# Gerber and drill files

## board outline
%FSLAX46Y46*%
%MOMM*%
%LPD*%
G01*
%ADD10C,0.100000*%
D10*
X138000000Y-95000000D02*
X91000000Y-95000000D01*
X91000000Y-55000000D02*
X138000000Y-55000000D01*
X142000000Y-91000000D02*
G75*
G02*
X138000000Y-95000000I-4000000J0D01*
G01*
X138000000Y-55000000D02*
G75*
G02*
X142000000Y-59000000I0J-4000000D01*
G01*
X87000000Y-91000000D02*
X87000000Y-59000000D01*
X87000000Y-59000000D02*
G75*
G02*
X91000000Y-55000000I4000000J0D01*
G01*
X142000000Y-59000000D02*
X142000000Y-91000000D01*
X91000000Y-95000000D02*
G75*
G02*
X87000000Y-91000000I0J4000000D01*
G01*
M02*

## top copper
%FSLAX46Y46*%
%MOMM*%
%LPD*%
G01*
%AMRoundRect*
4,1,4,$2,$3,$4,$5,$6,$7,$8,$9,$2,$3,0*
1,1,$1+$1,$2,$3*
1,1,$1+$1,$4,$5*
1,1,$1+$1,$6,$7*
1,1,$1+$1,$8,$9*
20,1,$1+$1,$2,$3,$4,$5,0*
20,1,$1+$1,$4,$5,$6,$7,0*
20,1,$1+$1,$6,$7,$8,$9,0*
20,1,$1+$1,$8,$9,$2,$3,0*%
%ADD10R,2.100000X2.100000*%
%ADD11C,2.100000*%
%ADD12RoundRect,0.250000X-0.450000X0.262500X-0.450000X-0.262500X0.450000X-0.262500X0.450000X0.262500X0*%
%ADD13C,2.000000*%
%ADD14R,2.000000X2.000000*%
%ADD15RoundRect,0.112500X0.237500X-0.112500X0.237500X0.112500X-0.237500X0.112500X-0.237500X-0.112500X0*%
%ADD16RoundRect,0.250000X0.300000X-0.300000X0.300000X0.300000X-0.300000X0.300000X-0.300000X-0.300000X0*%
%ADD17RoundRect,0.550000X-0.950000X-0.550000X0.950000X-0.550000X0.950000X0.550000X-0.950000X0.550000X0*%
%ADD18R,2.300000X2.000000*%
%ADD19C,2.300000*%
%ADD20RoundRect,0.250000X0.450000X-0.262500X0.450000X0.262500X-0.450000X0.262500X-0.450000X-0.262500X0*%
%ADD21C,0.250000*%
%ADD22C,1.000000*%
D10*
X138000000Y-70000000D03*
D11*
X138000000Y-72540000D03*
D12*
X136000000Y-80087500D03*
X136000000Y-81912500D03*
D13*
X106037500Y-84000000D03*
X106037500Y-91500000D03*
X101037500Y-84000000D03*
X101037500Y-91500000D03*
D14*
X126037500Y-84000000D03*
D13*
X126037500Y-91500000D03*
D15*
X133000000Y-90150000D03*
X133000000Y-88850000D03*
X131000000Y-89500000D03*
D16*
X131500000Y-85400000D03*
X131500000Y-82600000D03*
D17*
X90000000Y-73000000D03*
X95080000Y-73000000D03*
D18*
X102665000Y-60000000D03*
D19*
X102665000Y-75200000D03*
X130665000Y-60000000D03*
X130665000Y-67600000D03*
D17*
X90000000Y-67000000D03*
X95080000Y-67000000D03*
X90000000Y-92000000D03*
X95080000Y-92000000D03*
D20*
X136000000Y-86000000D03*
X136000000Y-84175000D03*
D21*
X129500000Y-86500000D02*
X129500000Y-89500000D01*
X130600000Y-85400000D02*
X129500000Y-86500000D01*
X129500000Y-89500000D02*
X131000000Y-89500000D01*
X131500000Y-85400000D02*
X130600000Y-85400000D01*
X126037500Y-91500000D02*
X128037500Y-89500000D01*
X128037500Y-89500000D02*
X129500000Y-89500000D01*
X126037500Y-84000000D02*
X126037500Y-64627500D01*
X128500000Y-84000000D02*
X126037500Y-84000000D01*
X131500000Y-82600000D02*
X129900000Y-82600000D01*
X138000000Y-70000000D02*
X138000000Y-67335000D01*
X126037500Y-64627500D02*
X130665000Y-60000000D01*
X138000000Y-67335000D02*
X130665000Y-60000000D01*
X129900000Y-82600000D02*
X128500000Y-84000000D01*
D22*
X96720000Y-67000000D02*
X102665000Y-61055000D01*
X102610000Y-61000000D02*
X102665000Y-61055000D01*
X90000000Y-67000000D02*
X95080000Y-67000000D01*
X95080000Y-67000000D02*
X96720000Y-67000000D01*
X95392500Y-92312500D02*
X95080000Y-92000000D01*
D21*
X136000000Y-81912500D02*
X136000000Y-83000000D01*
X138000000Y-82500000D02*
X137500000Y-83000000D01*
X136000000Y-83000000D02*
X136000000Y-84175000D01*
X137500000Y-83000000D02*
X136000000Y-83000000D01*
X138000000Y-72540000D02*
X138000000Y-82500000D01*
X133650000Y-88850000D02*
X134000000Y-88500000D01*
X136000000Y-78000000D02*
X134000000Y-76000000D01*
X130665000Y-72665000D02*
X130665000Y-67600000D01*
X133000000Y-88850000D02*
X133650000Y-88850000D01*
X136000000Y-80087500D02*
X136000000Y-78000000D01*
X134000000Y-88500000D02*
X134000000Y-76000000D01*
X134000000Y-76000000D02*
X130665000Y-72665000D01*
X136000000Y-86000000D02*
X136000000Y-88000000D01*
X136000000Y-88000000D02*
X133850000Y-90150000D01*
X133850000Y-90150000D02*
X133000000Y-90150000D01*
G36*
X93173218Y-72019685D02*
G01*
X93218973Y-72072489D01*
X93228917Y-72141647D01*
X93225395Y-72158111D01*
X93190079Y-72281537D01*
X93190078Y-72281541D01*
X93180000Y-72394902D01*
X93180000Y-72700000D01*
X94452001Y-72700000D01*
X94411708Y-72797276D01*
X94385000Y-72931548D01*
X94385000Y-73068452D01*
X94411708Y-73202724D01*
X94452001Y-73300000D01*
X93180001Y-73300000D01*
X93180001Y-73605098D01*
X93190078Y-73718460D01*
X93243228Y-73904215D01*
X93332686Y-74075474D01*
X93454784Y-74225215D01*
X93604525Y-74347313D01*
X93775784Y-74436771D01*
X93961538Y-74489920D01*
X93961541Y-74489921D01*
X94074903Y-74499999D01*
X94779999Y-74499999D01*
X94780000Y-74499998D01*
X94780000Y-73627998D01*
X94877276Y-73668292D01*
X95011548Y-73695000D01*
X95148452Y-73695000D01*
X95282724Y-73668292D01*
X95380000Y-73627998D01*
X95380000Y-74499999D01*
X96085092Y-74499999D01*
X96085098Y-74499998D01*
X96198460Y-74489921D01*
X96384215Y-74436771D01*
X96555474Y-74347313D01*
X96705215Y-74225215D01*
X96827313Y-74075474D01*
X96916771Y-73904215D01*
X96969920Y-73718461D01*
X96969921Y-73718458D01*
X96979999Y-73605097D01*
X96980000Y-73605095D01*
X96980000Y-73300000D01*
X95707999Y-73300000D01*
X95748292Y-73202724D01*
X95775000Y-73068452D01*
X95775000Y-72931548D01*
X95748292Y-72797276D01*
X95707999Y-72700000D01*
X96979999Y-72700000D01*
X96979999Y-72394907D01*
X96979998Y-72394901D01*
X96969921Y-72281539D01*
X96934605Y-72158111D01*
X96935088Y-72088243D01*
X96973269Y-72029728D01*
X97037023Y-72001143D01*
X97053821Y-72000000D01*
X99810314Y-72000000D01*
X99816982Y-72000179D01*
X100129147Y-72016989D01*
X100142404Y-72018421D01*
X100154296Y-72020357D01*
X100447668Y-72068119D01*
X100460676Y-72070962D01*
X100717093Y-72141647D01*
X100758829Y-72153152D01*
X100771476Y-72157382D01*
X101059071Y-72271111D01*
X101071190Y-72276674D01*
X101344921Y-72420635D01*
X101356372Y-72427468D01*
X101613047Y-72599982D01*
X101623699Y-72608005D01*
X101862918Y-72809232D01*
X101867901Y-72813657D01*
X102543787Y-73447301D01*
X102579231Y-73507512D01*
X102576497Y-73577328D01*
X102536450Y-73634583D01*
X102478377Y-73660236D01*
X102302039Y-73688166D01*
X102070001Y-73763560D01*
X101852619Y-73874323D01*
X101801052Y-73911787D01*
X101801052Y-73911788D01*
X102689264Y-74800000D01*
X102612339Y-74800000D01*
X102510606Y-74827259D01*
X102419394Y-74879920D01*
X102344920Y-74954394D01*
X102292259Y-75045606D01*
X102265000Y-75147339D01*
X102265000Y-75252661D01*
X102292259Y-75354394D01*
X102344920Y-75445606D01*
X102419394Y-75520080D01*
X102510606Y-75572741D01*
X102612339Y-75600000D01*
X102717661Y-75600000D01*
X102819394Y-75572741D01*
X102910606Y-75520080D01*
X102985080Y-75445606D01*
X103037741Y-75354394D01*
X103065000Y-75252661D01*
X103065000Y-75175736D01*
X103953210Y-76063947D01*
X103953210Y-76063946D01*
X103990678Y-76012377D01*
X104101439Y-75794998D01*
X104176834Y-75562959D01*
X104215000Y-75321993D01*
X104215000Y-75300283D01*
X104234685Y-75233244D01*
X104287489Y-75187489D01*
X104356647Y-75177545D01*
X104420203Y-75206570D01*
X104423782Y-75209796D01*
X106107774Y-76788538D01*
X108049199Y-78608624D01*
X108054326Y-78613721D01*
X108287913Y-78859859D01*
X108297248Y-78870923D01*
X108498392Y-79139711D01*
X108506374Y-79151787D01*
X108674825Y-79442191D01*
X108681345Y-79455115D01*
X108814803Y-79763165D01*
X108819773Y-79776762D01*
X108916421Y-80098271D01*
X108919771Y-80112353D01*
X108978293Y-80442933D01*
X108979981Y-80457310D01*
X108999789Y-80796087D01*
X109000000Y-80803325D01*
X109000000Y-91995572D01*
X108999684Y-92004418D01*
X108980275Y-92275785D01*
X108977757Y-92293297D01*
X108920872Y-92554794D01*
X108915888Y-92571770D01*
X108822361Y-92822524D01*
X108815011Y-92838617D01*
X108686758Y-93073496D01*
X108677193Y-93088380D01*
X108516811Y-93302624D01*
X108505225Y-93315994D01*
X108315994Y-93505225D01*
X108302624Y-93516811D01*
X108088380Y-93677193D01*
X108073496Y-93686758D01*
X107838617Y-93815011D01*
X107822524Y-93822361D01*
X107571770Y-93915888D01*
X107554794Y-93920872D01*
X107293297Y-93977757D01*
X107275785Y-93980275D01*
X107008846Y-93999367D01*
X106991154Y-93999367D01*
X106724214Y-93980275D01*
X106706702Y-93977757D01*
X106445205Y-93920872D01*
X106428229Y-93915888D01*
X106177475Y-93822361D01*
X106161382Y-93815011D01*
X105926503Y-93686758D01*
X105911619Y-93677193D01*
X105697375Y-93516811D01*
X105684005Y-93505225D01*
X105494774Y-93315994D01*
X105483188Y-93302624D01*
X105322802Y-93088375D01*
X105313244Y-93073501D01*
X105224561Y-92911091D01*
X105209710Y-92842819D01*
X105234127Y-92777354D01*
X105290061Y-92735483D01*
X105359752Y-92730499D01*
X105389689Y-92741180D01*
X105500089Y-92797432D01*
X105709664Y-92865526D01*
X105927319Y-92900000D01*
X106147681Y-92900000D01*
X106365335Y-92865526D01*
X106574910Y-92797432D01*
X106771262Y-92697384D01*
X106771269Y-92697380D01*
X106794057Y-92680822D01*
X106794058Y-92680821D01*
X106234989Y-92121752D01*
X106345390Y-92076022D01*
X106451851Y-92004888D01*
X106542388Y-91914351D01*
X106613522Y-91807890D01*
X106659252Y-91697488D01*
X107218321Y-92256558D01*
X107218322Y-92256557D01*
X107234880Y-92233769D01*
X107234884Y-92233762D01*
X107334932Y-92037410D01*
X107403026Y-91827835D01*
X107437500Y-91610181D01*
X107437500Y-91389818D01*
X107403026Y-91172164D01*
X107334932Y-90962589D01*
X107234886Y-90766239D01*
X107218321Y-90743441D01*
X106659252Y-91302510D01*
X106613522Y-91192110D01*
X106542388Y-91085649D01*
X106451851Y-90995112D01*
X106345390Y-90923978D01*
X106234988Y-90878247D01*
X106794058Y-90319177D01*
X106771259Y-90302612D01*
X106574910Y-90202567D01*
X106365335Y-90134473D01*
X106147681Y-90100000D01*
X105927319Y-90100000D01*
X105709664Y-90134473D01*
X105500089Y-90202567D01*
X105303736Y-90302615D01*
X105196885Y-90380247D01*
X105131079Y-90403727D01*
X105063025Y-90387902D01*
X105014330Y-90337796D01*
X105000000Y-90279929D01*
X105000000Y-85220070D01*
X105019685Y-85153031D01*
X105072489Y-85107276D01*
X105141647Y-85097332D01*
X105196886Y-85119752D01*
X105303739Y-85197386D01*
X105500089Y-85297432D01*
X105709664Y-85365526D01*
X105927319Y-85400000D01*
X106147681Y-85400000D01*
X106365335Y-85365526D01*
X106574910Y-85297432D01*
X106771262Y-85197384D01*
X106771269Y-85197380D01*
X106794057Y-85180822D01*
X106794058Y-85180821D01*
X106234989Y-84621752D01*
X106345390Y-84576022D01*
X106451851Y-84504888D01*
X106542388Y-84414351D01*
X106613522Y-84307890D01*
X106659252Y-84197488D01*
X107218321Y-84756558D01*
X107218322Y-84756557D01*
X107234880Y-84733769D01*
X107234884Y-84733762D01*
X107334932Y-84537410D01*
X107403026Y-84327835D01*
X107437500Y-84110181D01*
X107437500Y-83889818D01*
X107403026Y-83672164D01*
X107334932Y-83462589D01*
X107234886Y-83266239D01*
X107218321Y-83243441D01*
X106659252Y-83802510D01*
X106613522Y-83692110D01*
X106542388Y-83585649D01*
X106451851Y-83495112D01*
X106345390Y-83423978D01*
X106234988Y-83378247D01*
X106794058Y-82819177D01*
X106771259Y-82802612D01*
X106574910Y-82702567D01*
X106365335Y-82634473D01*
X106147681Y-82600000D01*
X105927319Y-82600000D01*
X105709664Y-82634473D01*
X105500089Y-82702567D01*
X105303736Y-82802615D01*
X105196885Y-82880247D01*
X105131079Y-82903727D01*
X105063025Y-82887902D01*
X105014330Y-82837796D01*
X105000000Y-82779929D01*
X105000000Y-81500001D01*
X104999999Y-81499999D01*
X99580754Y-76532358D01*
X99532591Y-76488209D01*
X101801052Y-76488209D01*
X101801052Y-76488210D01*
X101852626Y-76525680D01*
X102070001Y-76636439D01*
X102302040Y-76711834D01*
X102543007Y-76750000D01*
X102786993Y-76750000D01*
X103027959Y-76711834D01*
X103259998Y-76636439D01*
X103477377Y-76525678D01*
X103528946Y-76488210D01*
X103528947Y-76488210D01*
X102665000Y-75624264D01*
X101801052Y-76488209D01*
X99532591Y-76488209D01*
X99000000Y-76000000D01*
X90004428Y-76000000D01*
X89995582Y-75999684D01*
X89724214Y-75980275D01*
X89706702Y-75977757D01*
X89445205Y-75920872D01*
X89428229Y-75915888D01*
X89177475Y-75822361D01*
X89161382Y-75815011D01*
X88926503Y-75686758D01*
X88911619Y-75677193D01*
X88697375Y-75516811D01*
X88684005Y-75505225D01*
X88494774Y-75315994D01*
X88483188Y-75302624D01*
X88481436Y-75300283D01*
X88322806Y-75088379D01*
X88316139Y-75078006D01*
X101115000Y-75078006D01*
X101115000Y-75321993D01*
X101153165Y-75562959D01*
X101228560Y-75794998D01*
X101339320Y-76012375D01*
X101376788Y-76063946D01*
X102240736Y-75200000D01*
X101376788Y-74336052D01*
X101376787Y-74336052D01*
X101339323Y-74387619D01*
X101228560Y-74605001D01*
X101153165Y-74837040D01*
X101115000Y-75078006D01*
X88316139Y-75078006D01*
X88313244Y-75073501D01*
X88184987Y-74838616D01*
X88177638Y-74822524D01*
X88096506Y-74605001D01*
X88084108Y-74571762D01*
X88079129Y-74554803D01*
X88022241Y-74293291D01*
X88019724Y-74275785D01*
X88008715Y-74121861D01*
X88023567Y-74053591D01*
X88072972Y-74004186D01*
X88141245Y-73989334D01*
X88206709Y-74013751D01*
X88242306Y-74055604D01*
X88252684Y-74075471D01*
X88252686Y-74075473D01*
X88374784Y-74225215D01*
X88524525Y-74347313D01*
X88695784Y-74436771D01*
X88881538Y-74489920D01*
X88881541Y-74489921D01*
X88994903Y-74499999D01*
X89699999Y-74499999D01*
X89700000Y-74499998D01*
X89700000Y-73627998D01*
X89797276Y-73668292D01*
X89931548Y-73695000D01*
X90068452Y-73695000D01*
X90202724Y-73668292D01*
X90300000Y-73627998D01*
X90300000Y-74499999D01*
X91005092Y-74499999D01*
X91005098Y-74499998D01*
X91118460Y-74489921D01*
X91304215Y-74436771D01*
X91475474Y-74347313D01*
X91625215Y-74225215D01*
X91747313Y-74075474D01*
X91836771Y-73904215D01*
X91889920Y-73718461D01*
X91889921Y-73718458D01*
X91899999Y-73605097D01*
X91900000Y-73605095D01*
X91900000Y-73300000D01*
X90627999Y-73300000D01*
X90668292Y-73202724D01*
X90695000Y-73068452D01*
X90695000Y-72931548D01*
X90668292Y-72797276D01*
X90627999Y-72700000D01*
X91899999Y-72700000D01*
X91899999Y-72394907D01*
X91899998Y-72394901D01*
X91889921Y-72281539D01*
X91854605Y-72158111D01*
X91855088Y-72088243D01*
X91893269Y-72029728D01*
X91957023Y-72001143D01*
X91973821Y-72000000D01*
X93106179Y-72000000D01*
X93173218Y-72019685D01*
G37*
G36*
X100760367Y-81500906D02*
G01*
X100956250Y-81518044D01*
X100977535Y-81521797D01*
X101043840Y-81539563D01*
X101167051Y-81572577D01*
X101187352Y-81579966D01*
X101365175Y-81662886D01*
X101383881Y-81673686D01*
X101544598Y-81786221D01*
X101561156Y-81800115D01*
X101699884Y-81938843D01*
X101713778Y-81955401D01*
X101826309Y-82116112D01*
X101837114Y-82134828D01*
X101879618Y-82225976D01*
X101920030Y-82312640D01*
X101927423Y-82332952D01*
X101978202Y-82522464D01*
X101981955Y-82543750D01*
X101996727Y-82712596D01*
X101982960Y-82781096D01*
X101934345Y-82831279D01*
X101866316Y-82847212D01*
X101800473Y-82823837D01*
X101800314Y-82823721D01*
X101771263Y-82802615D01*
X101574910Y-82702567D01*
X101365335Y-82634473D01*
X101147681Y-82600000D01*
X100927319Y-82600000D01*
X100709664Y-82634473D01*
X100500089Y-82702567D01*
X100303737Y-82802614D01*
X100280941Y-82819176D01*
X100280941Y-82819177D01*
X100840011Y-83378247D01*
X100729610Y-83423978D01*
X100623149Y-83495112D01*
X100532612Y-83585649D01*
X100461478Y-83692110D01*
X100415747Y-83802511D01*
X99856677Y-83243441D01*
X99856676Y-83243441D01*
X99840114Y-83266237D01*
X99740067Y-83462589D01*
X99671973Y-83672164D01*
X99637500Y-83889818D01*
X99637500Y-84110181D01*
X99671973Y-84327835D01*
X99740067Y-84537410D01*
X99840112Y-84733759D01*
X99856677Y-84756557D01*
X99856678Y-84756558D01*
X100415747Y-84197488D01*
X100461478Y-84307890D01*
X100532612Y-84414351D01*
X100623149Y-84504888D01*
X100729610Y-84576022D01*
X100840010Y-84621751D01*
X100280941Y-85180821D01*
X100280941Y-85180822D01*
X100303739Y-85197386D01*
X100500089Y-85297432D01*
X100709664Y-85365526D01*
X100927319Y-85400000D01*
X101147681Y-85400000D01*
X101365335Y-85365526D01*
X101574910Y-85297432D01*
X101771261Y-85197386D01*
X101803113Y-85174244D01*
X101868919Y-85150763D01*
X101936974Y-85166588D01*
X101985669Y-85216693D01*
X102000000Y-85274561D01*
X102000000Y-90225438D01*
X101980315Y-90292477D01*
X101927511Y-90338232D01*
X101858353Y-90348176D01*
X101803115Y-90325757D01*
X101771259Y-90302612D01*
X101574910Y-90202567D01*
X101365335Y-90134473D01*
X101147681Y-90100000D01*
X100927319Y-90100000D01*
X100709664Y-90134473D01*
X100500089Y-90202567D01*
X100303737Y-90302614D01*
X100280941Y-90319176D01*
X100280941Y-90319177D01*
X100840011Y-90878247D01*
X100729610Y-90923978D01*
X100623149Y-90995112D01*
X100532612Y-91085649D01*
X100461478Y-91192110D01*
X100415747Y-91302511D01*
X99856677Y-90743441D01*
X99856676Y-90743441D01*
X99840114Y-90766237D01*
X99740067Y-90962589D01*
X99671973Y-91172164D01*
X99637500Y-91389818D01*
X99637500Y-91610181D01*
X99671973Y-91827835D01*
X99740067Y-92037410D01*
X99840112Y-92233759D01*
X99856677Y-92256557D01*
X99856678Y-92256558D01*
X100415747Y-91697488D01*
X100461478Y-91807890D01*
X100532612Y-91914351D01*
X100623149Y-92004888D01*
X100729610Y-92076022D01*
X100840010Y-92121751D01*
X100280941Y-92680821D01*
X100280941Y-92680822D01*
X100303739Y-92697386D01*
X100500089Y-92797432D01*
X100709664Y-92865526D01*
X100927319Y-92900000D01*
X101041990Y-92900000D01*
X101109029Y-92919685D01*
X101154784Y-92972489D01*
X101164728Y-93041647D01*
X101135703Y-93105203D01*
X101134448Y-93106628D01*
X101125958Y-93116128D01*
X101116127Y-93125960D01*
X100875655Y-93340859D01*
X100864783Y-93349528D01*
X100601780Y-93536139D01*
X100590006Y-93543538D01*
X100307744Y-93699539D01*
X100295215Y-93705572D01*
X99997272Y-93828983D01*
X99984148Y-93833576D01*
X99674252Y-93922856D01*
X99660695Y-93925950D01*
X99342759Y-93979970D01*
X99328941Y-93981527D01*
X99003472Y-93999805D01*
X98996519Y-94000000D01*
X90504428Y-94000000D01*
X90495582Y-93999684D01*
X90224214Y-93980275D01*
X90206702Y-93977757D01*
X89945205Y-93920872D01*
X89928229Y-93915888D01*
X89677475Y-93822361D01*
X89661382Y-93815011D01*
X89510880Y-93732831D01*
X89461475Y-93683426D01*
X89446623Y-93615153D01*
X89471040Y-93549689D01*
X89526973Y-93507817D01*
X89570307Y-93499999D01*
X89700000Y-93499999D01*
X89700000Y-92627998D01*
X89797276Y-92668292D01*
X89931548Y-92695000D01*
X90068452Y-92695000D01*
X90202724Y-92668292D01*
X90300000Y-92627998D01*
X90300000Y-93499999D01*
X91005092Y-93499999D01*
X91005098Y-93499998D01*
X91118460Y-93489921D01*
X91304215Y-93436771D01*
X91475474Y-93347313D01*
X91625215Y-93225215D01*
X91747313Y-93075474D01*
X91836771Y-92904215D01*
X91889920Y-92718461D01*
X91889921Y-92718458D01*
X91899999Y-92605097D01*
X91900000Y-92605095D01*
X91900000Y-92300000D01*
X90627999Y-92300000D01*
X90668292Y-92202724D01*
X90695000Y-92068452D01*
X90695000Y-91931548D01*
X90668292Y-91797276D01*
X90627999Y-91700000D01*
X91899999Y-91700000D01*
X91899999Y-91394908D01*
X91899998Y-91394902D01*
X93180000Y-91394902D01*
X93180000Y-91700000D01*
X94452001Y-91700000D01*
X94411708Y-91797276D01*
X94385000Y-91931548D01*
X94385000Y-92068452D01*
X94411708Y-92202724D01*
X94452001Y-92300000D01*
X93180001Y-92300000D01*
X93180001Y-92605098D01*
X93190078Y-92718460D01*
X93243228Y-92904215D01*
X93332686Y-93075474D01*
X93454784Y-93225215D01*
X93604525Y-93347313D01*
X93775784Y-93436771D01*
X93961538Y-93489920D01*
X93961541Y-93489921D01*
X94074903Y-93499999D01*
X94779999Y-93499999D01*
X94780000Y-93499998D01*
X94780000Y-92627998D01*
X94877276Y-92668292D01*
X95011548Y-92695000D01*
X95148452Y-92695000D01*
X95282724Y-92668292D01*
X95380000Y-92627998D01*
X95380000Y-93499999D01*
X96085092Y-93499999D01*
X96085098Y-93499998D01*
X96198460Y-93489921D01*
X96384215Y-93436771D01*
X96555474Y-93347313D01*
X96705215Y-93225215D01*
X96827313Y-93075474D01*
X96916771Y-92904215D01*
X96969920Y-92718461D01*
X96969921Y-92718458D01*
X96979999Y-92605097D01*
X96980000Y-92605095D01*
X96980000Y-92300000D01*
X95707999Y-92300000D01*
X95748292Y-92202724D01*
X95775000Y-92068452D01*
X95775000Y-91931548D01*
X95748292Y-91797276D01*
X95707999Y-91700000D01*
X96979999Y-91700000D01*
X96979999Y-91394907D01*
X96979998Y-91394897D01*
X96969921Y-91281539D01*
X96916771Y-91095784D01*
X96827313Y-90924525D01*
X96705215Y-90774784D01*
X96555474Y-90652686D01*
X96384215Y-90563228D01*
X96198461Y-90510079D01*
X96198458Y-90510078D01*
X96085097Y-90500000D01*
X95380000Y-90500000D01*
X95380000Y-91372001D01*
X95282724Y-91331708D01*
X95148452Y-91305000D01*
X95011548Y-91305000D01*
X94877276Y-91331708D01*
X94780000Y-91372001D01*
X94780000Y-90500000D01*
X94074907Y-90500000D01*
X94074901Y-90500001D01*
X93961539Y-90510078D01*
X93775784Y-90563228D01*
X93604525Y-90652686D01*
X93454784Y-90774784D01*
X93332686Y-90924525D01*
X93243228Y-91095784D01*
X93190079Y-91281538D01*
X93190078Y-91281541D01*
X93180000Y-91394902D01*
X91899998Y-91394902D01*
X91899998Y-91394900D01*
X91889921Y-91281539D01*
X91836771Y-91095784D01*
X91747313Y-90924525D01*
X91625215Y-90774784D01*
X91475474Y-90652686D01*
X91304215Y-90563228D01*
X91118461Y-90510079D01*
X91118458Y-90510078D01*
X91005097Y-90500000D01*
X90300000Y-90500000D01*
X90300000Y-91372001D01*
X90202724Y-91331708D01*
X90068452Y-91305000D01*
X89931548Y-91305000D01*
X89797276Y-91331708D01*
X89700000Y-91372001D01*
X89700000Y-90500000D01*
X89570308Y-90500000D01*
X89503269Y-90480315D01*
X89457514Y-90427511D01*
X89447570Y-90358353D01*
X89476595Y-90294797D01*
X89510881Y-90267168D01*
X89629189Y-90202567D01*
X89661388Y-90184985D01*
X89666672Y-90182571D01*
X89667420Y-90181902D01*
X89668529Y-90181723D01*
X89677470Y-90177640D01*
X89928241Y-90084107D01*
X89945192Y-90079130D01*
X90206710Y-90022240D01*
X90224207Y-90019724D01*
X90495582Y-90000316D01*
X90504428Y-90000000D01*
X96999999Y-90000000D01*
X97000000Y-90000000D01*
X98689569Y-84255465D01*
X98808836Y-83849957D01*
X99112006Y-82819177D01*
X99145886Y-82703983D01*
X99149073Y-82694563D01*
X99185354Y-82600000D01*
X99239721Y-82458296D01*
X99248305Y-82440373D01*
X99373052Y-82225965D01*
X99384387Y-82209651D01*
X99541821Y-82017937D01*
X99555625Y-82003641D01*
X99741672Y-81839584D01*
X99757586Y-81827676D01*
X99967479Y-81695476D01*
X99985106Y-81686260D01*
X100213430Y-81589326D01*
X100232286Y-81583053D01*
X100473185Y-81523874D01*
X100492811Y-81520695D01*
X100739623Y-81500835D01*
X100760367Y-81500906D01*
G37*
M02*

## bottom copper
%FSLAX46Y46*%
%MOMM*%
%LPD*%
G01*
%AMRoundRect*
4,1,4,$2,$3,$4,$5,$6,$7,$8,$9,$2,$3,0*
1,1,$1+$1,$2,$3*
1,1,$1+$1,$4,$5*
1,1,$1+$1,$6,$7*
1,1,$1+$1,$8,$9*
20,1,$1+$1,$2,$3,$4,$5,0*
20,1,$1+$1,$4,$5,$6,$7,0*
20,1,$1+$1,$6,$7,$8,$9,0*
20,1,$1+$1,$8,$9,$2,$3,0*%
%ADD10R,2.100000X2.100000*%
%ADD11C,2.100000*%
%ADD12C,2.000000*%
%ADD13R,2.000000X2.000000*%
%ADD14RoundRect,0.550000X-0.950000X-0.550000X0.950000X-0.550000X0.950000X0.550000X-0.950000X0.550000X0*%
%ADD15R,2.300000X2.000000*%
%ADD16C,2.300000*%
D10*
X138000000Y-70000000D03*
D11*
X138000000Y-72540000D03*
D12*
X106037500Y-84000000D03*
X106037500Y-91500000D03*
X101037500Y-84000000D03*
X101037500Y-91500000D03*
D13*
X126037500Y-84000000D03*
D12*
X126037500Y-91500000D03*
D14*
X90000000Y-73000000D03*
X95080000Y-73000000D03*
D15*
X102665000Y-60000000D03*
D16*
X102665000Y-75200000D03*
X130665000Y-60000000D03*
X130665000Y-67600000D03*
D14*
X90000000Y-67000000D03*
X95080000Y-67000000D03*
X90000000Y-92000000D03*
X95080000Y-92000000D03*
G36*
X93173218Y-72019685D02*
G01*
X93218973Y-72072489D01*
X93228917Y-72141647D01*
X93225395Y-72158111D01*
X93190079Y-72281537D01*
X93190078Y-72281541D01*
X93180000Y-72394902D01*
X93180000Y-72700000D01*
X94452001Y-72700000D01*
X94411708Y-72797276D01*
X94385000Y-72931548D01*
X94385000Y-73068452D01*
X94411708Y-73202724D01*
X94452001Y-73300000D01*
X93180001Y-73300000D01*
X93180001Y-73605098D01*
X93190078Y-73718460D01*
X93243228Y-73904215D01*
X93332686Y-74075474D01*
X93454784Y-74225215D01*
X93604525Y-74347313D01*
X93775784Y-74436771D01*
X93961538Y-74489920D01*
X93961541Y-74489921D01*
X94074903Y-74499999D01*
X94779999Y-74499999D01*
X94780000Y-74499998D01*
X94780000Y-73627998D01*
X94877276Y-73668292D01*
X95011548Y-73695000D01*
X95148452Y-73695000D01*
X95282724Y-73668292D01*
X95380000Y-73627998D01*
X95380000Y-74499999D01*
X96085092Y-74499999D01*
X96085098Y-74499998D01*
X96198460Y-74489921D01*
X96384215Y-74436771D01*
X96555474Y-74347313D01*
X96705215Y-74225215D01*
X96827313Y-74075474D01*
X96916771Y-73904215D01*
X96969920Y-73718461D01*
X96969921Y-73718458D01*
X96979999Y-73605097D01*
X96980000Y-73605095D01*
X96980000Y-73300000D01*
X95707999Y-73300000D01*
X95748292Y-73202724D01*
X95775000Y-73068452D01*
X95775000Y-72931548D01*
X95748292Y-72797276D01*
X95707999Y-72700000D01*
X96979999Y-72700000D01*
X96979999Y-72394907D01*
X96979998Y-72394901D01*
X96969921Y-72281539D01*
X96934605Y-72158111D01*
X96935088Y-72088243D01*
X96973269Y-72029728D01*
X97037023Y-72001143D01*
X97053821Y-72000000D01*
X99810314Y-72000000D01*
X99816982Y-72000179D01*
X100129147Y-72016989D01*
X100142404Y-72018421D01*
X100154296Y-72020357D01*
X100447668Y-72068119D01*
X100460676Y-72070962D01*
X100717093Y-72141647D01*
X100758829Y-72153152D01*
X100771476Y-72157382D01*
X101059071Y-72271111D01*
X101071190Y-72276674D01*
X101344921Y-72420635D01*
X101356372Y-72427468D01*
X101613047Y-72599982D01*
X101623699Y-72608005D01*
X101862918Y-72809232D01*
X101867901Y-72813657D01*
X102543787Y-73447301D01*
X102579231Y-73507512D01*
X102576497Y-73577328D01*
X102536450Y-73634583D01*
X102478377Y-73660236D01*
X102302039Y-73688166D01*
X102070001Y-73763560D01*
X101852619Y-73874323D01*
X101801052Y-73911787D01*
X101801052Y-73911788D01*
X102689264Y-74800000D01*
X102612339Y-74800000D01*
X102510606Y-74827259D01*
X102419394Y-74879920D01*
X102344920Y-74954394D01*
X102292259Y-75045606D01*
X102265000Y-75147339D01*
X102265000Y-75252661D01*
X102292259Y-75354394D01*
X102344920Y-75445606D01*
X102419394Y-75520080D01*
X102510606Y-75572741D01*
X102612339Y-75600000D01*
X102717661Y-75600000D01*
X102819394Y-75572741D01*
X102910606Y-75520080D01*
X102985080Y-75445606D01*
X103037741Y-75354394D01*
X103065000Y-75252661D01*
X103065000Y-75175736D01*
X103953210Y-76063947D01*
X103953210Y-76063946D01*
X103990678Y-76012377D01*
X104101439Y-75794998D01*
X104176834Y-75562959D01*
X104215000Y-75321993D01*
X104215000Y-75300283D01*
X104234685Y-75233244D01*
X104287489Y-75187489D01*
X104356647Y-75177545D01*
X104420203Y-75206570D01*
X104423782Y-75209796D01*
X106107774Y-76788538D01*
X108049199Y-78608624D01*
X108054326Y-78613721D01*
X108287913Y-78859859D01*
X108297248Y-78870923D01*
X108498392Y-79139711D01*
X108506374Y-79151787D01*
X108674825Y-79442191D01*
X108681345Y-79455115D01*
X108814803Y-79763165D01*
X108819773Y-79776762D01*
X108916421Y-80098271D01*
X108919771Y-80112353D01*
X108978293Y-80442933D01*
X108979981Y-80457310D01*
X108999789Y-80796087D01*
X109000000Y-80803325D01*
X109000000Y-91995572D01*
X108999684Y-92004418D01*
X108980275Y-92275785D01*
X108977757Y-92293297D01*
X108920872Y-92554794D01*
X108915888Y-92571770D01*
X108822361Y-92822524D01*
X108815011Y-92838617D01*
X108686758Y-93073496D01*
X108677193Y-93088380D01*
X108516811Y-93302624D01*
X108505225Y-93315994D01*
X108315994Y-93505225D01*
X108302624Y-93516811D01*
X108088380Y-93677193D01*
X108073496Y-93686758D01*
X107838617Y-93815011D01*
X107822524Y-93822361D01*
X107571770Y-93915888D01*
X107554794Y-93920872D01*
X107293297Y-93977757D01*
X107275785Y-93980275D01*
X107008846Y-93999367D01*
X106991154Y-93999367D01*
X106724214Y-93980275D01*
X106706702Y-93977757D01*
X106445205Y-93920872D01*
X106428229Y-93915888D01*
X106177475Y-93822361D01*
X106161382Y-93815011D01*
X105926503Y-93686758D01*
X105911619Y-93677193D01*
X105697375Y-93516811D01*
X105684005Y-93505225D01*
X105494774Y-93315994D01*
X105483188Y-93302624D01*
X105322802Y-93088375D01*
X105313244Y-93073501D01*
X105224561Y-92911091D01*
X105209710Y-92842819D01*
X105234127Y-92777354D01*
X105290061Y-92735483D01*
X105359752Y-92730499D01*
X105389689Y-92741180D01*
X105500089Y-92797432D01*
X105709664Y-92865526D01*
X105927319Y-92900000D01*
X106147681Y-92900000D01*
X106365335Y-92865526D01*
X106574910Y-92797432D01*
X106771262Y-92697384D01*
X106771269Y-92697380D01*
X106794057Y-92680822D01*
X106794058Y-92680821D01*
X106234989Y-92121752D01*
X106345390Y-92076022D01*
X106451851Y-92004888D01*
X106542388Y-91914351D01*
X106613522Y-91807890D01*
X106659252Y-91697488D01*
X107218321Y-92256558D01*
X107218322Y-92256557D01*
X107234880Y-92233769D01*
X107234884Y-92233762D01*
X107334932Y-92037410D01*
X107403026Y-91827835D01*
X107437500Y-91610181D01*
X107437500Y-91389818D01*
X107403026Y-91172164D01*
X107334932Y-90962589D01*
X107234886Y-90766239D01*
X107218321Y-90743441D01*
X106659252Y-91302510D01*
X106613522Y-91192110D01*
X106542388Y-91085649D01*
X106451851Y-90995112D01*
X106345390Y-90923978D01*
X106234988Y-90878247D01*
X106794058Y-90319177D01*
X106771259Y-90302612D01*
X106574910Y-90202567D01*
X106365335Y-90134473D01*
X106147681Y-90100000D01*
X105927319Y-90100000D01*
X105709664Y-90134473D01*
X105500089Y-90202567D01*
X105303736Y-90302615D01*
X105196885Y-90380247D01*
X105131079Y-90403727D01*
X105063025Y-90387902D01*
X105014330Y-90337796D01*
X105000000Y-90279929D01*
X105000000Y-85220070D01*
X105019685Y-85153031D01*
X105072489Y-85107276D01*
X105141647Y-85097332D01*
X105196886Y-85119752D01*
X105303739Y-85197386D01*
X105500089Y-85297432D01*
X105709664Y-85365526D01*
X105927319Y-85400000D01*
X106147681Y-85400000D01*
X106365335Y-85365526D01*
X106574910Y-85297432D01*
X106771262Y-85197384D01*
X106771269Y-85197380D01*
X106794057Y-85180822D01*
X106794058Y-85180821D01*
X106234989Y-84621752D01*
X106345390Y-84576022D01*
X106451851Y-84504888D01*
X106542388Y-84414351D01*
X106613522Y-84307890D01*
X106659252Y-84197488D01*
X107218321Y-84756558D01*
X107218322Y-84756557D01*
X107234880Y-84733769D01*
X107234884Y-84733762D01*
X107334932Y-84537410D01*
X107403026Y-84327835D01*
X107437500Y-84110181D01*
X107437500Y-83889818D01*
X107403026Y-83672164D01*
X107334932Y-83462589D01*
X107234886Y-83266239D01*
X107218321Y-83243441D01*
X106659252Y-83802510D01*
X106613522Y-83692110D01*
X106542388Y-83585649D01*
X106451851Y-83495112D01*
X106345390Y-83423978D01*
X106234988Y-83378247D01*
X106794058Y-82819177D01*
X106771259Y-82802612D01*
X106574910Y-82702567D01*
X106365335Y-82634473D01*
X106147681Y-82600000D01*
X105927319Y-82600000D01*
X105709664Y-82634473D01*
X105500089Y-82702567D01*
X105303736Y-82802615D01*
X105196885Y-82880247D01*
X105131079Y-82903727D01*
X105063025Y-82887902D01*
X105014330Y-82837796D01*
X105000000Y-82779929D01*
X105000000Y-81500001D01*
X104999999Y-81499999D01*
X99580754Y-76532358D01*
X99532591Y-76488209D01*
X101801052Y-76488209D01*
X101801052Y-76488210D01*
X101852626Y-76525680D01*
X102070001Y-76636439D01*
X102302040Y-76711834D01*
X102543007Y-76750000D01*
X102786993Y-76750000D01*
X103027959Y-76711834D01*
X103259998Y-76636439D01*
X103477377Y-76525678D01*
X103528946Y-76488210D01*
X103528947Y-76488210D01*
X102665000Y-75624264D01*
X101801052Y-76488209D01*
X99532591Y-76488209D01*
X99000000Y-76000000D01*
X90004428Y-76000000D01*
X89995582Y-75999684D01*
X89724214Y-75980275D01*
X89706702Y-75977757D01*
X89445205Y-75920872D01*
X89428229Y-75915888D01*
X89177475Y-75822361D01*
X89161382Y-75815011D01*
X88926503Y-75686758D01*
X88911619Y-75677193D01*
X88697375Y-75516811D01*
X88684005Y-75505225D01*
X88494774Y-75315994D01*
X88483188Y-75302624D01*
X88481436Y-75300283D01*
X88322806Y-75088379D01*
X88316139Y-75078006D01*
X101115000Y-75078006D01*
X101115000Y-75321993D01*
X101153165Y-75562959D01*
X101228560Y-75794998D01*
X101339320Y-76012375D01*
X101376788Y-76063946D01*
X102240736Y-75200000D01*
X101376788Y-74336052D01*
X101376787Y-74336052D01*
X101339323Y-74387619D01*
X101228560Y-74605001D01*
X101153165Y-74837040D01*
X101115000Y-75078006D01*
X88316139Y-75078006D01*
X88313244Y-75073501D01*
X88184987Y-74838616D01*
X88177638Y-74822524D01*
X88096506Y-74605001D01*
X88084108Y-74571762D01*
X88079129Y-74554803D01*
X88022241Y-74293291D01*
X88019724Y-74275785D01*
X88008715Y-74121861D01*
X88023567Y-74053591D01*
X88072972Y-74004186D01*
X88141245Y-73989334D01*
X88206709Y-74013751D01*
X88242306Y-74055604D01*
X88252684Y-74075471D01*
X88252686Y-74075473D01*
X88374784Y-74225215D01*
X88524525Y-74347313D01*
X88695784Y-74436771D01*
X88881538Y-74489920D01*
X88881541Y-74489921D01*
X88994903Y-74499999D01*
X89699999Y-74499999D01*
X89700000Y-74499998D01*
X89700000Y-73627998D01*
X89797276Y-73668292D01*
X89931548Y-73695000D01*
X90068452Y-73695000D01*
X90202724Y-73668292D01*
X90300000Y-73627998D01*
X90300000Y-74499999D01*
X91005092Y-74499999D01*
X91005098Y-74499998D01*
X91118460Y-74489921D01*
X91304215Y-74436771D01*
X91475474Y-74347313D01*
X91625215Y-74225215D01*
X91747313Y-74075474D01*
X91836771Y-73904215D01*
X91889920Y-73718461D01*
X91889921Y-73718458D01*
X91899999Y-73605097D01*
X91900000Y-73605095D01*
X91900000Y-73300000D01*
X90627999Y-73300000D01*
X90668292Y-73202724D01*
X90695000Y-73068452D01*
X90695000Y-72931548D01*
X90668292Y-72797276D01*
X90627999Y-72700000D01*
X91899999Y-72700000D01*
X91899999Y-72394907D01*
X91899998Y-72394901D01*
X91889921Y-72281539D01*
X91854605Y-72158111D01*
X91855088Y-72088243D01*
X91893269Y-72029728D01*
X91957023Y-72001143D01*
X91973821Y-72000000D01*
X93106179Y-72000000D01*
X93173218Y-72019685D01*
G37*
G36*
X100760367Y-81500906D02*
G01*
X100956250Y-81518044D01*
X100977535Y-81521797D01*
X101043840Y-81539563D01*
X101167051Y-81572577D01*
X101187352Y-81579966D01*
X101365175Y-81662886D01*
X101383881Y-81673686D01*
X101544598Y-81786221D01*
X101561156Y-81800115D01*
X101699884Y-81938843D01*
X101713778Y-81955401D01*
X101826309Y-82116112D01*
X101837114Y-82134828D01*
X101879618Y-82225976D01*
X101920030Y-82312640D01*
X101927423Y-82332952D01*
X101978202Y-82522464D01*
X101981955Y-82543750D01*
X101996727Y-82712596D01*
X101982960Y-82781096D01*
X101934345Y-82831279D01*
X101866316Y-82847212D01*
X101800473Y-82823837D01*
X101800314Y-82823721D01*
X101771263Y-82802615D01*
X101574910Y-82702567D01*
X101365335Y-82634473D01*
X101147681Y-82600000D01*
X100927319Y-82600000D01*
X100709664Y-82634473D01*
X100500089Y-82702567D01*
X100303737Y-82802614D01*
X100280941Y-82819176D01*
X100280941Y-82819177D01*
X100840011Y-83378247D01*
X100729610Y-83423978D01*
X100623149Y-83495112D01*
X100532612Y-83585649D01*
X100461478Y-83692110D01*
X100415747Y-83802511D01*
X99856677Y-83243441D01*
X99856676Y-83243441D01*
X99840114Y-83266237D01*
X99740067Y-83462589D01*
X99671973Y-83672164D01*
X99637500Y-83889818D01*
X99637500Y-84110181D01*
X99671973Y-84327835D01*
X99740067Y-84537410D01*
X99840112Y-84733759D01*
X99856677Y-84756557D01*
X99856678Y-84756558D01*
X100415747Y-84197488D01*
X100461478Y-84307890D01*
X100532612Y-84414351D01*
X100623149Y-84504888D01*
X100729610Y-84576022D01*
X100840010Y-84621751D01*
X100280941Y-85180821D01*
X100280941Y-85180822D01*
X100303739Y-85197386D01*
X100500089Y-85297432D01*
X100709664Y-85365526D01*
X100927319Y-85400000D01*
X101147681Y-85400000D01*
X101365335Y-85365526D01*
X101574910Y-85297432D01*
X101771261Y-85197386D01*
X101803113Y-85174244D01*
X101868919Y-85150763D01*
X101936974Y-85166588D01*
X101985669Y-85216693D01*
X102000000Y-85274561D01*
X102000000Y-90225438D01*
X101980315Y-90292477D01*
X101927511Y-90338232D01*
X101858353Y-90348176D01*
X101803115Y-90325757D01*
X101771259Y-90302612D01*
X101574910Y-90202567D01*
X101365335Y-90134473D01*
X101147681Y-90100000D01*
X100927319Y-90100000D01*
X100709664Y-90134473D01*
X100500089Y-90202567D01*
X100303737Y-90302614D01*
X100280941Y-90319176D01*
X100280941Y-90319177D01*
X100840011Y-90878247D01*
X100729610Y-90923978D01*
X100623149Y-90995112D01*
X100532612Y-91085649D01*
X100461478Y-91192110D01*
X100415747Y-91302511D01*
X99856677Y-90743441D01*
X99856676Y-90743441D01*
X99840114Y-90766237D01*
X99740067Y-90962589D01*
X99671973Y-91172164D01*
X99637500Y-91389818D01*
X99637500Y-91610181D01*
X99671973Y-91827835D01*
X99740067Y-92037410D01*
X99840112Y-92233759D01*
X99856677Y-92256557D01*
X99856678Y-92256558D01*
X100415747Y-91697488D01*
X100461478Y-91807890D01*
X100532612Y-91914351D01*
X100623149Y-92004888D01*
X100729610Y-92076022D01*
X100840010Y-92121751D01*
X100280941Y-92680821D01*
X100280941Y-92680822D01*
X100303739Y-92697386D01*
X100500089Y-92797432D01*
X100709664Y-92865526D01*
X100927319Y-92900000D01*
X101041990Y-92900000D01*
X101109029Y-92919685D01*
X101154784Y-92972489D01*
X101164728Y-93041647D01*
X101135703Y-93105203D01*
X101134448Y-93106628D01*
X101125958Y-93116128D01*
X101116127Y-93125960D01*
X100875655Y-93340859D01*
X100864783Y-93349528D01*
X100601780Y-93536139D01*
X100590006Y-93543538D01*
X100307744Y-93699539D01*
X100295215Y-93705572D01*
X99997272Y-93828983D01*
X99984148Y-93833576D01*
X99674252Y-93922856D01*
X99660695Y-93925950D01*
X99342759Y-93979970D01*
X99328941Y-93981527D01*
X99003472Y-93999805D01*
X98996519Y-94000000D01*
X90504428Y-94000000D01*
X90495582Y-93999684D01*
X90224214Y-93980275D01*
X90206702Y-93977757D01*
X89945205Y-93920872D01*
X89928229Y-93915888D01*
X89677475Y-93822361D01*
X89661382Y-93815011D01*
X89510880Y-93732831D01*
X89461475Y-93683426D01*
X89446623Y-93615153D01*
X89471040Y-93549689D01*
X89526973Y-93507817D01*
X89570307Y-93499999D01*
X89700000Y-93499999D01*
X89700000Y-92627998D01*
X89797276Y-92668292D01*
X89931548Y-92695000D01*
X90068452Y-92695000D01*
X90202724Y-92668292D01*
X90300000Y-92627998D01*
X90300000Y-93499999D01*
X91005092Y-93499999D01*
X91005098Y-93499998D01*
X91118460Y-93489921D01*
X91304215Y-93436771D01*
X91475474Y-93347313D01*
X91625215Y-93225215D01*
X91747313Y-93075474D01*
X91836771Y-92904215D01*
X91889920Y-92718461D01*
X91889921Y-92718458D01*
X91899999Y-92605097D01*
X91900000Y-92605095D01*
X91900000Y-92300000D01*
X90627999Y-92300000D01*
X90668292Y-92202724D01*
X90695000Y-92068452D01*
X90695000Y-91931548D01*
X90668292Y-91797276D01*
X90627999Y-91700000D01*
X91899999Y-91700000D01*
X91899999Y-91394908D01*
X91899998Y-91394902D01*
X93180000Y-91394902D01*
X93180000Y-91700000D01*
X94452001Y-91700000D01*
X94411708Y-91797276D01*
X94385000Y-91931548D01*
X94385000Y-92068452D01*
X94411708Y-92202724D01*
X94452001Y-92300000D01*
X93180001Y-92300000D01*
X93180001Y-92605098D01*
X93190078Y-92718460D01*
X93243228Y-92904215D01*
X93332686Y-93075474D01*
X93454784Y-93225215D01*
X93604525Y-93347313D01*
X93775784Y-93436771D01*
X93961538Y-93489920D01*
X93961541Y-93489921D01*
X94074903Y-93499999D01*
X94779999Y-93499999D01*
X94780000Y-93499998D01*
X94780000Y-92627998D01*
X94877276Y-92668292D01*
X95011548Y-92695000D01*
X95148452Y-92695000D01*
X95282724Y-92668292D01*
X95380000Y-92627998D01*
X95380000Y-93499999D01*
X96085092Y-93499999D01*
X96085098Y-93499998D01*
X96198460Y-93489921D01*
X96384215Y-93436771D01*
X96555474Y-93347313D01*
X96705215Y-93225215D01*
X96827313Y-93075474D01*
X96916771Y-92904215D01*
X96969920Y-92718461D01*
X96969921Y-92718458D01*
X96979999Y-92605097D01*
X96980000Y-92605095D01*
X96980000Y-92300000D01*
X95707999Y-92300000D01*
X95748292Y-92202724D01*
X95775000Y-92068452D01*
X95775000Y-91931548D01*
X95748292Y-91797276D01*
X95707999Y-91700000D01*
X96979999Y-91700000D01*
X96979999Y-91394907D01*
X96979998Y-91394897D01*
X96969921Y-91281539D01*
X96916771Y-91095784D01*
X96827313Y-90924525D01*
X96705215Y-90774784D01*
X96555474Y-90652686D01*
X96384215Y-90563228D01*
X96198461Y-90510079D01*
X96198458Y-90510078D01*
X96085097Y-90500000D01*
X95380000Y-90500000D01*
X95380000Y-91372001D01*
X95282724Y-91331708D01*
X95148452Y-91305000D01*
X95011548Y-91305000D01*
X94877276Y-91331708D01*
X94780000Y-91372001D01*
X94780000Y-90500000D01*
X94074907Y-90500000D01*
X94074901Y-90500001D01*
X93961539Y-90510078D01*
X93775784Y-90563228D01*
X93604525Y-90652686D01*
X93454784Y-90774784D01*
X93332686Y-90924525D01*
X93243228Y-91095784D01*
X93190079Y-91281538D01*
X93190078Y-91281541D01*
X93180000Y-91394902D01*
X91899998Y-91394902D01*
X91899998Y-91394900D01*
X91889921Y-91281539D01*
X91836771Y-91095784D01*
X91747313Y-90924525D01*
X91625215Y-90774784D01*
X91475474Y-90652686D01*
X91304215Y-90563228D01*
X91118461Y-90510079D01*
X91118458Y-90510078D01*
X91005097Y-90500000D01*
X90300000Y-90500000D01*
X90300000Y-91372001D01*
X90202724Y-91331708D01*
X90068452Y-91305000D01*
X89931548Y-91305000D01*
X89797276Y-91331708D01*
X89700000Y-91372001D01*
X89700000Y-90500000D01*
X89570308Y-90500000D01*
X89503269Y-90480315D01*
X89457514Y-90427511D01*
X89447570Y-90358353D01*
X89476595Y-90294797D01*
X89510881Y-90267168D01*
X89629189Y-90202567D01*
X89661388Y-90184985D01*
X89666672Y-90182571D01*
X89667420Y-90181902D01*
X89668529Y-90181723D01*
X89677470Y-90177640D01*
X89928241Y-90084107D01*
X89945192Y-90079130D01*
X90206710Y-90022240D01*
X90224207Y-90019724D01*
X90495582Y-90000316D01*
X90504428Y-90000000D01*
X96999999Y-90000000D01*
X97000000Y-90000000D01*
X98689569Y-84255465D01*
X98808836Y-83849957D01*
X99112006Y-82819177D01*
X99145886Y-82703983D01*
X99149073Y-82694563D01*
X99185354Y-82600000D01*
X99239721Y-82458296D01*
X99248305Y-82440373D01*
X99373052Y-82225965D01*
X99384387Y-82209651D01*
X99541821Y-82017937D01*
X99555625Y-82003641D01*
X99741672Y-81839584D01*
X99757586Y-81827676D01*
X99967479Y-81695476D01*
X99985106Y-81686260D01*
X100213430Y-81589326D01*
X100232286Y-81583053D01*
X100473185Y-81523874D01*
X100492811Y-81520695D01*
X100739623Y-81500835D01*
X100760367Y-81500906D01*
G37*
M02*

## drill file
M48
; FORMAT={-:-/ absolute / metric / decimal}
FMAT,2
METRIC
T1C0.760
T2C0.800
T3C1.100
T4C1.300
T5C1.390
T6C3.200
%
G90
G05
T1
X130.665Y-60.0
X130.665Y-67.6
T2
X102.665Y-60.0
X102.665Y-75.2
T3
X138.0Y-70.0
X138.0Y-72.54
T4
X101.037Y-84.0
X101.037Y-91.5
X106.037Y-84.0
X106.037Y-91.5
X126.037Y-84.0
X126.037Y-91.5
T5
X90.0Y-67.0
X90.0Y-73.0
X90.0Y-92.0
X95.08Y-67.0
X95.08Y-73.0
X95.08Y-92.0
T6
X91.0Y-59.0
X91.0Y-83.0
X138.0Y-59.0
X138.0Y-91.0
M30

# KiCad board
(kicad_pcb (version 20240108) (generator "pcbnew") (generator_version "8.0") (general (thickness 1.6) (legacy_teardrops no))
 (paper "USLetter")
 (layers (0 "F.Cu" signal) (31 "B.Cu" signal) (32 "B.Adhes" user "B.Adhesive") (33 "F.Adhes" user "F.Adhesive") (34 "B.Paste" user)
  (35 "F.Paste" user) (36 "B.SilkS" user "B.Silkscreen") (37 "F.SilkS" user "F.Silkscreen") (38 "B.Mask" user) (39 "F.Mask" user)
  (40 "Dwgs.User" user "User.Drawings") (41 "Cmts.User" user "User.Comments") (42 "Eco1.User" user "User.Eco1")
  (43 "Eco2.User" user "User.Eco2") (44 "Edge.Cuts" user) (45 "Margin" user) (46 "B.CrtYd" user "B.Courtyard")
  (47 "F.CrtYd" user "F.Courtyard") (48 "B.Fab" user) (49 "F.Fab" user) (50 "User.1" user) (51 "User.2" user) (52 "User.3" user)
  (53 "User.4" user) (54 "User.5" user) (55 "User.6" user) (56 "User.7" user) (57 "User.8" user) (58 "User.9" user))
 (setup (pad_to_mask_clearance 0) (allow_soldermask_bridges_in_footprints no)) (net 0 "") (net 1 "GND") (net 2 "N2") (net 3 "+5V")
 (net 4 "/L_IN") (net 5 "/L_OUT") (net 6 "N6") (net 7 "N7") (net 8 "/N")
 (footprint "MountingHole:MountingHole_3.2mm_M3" (layer "F.Cu") (at 138 59)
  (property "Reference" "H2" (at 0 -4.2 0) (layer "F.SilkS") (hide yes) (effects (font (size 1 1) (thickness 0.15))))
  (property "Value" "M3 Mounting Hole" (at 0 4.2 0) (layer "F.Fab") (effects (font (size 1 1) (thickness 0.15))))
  (pad "" np_thru_hole circle (at 0 0) (size 3.2 3.2) (drill 3.2) (layers "*.Cu" "*.Mask")))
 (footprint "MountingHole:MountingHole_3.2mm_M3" (layer "F.Cu") (at 138 91)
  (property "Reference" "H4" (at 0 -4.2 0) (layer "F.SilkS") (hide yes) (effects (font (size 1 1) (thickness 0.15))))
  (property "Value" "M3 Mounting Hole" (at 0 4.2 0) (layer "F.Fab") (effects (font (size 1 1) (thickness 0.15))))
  (pad "" np_thru_hole circle (at 0 0) (size 3.2 3.2) (drill 3.2) (layers "*.Cu" "*.Mask")))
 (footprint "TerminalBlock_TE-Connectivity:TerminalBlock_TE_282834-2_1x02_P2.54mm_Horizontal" (layer "F.Cu") (at 138 70 -90)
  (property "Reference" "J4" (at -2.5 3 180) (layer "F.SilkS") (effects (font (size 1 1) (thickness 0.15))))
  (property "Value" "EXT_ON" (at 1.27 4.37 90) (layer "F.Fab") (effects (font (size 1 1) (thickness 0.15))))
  (pad "1" thru_hole rect (at 0 0 270) (size 2.1 2.1) (drill 1.1) (layers "*.Cu" "*.Mask") (remove_unused_layers no) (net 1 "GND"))
  (pad "2" thru_hole circle (at 2.54 0 270) (size 2.1 2.1) (drill 1.1) (layers "*.Cu" "*.Mask") (remove_unused_layers no) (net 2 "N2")))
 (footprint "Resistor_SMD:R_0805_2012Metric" (layer "F.Cu") (at 136 81 -90)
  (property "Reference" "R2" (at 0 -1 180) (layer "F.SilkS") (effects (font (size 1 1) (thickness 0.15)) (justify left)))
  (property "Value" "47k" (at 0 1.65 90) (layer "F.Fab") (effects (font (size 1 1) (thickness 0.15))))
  (pad "1" smd roundrect (at -0.9125 0 270) (size 1.025 1.4) (layers "F.Cu" "F.Paste" "F.Mask") (roundrect_rratio 0.243902439) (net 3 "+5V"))
  (pad "2" smd roundrect (at 0.9125 0 270) (size 1.025 1.4) (layers "F.Cu" "F.Paste" "F.Mask") (roundrect_rratio 0.243902439) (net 2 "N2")))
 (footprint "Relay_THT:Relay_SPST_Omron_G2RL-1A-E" (layer "F.Cu") (at 126.0375 84 -90)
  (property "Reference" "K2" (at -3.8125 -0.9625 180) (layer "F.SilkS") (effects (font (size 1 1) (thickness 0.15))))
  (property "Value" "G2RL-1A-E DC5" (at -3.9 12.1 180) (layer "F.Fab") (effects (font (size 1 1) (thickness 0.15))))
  (pad "13" thru_hole circle (at 0 20 270) (size 2 2) (drill 1.3) (layers "*.Cu" "*.Mask") (remove_unused_layers no) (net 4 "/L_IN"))
  (pad "13" thru_hole circle (at 7.5 20 270) (size 2 2) (drill 1.3) (layers "*.Cu" "*.Mask") (remove_unused_layers no) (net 4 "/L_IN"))
  (pad "14" thru_hole circle (at 0 25 270) (size 2 2) (drill 1.3) (layers "*.Cu" "*.Mask") (remove_unused_layers no) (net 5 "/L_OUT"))
  (pad "14" thru_hole circle (at 7.5 25 270) (size 2 2) (drill 1.3) (layers "*.Cu" "*.Mask") (remove_unused_layers no) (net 5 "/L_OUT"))
  (pad "A1" thru_hole rect (at 0 0 270) (size 2 2) (drill 1.3) (layers "*.Cu" "*.Mask") (remove_unused_layers no) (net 1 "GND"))
  (pad "A2" thru_hole circle (at 7.5 0 270) (size 2 2) (drill 1.3) (layers "*.Cu" "*.Mask") (remove_unused_layers no) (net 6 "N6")))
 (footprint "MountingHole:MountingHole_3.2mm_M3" (layer "F.Cu") (at 91 59)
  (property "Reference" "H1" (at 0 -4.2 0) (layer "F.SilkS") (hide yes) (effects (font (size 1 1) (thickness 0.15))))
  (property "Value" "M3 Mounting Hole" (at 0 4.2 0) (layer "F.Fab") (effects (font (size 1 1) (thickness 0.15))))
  (pad "" np_thru_hole circle (at 0 0) (size 3.2 3.2) (drill 3.2) (layers "*.Cu" "*.Mask")))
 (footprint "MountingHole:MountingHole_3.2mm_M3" (layer "F.Cu") (at 91 83)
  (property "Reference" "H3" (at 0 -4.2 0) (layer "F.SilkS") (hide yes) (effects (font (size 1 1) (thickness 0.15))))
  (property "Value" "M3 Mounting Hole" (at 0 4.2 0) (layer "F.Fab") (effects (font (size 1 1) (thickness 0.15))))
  (pad "" np_thru_hole circle (at 0 0) (size 3.2 3.2) (drill 3.2) (layers "*.Cu" "*.Mask")))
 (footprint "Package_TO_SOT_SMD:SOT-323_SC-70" (layer "F.Cu") (at 132 89.5 180)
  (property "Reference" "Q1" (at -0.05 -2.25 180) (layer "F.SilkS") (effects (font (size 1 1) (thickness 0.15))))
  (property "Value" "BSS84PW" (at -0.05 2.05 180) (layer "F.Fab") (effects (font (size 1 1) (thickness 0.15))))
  (pad "1" smd roundrect (at -1 -0.65 90) (size 0.45 0.7) (layers "F.Cu" "F.Paste" "F.Mask") (roundrect_rratio 0.25) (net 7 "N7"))
  (pad "2" smd roundrect (at -1 0.65 90) (size 0.45 0.7) (layers "F.Cu" "F.Paste" "F.Mask") (roundrect_rratio 0.25) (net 3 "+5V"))
  (pad "3" smd roundrect (at 1 0 90) (size 0.45 0.7) (layers "F.Cu" "F.Paste" "F.Mask") (roundrect_rratio 0.25) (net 6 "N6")))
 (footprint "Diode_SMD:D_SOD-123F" (layer "F.Cu") (at 131.5 84 90)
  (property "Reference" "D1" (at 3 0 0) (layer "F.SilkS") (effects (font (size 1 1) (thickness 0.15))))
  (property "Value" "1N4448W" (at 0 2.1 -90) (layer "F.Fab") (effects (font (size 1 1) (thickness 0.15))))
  (pad "1" smd roundrect (at -1.4 0 90) (size 1.1 1.1) (layers "F.Cu" "F.Paste" "F.Mask") (roundrect_rratio 0.2272727273) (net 6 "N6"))
  (pad "2" smd roundrect (at 1.4 0 90) (size 1.1 1.1) (layers "F.Cu" "F.Paste" "F.Mask") (roundrect_rratio 0.2272727273) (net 1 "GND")))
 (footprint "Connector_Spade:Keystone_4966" (layer "F.Cu") (at 92.54 73)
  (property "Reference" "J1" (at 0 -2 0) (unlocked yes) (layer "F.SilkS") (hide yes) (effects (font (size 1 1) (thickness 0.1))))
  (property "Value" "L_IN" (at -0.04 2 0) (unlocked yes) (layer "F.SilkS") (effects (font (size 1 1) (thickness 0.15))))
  (pad "1" thru_hole roundrect (at -2.54 0) (size 3 2.2) (drill 1.39) (layers "*.Cu" "*.Mask") (remove_unused_layers no)
   (roundrect_rratio 0.25) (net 4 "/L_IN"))
  (pad "1" thru_hole roundrect (at 2.54 0) (size 3 2.2) (drill 1.39) (layers "*.Cu" "*.Mask") (remove_unused_layers no)
   (roundrect_rratio 0.25) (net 4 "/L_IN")))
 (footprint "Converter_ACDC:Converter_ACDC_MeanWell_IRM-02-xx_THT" (layer "F.Cu") (at 102.665 60)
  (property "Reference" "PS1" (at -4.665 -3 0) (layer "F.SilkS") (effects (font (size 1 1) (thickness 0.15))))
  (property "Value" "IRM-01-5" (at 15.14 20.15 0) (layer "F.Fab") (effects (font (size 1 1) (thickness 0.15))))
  (pad "1" thru_hole rect (at 0 0) (size 2.3 2) (drill 0.8) (layers "*.Cu" "*.Mask") (remove_unused_layers no) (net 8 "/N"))
  (pad "2" thru_hole circle (at 0 15.2) (size 2.3 2.3) (drill 0.8) (layers "*.Cu" "*.Mask") (remove_unused_layers no) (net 4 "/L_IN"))
  (pad "3" thru_hole circle (at 28 0) (size 2.3 2.3) (drill 0.76) (layers "*.Cu" "*.Mask") (remove_unused_layers no) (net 1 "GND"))
  (pad "4" thru_hole circle (at 28 7.6) (size 2.3 2.3) (drill 0.76) (layers "*.Cu" "*.Mask") (remove_unused_layers no) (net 3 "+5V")))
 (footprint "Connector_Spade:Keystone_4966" (layer "F.Cu") (at 92.54 67)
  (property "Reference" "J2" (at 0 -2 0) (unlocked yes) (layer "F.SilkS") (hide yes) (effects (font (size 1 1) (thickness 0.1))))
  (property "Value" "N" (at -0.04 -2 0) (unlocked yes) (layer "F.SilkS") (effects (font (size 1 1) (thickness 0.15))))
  (pad "1" thru_hole roundrect (at -2.54 0) (size 3 2.2) (drill 1.39) (layers "*.Cu" "*.Mask") (remove_unused_layers no)
   (roundrect_rratio 0.25) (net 8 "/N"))
  (pad "1" thru_hole roundrect (at 2.54 0) (size 3 2.2) (drill 1.39) (layers "*.Cu" "*.Mask") (remove_unused_layers no)
   (roundrect_rratio 0.25) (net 8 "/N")))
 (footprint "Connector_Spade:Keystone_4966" (layer "F.Cu") (at 92.54 92)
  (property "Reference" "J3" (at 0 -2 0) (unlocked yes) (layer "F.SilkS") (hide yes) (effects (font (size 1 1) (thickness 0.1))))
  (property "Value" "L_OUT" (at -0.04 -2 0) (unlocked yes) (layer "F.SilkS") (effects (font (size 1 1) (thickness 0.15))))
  (pad "1" thru_hole roundrect (at -2.54 0) (size 3 2.2) (drill 1.39) (layers "*.Cu" "*.Mask") (remove_unused_layers no)
   (roundrect_rratio 0.25) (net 5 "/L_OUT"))
  (pad "1" thru_hole roundrect (at 2.54 0) (size 3 2.2) (drill 1.39) (layers "*.Cu" "*.Mask") (remove_unused_layers no)
   (roundrect_rratio 0.25) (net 5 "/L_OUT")))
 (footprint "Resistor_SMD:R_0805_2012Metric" (layer "F.Cu") (at 136 85.0875 90)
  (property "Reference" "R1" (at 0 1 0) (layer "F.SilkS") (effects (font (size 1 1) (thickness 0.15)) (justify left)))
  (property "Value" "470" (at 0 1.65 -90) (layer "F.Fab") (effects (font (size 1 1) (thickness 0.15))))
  (pad "1" smd roundrect (at -0.9125 0 90) (size 1.025 1.4) (layers "F.Cu" "F.Paste" "F.Mask") (roundrect_rratio 0.243902439) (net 7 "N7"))
  (pad "2" smd roundrect (at 0.9125 0 90) (size 1.025 1.4) (layers "F.Cu" "F.Paste" "F.Mask") (roundrect_rratio 0.243902439) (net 2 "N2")))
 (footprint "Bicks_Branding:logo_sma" (layer "B.Cu") (at 133.669334 82.603235 -90)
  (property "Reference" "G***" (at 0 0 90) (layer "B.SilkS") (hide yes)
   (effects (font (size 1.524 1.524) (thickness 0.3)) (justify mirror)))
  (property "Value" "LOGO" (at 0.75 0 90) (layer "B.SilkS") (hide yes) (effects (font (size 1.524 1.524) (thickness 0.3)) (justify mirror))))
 (gr_line (start 138 95) (end 91 95) (stroke (width 0.1) (type default)) (layer "Edge.Cuts"))
 (gr_line (start 91 55) (end 138 55) (stroke (width 0.1) (type default)) (layer "Edge.Cuts"))
 (gr_arc (start 142 91) (mid 140.828427 93.828427) (end 138 95) (stroke (width 0.1) (type default)) (layer "Edge.Cuts"))
 (gr_arc (start 138 55) (mid 140.828427 56.171573) (end 142 59) (stroke (width 0.1) (type default)) (layer "Edge.Cuts"))
 (gr_line (start 87 91) (end 87 59) (stroke (width 0.1) (type default)) (layer "Edge.Cuts"))
 (gr_arc (start 87 59) (mid 88.171573 56.171573) (end 91 55) (stroke (width 0.1) (type default)) (layer "Edge.Cuts"))
 (gr_line (start 142 59) (end 142 91) (stroke (width 0.1) (type default)) (layer "Edge.Cuts"))
 (gr_arc (start 91 95) (mid 88.171573 93.828427) (end 87 91) (stroke (width 0.1) (type default)) (layer "Edge.Cuts"))
 (segment (start 129.5 86.5) (end 129.5 89.5) (width 0.25) (layer "F.Cu") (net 6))
 (segment (start 130.6 85.4) (end 129.5 86.5) (width 0.25) (layer "F.Cu") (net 6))
 (segment (start 129.5 89.5) (end 131 89.5) (width 0.25) (layer "F.Cu") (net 6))
 (segment (start 131.5 85.4) (end 130.6 85.4) (width 0.25) (layer "F.Cu") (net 6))
 (segment (start 126.0375 91.5) (end 128.0375 89.5) (width 0.25) (layer "F.Cu") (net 6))
 (segment (start 128.0375 89.5) (end 129.5 89.5) (width 0.25) (layer "F.Cu") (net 6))
 (segment (start 126.0375 84) (end 126.0375 64.6275) (width 0.25) (layer "F.Cu") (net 1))
 (segment (start 128.5 84) (end 126.0375 84) (width 0.25) (layer "F.Cu") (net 1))
 (segment (start 131.5 82.6) (end 129.9 82.6) (width 0.25) (layer "F.Cu") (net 1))
 (segment (start 138 70) (end 138 67.335) (width 0.25) (layer "F.Cu") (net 1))
 (segment (start 126.0375 64.6275) (end 130.665 60) (width 0.25) (layer "F.Cu") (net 1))
 (segment (start 138 67.335) (end 130.665 60) (width 0.25) (layer "F.Cu") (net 1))
 (segment (start 129.9 82.6) (end 128.5 84) (width 0.25) (layer "F.Cu") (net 1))
 (segment (start 96.72 67) (end 102.665 61.055) (width 1) (layer "F.Cu") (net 8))
 (segment (start 102.61 61) (end 102.665 61.055) (width 1) (layer "F.Cu") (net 8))
 (segment (start 90 67) (end 95.08 67) (width 1) (layer "F.Cu") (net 8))
 (segment (start 95.08 67) (end 96.72 67) (width 1) (layer "F.Cu") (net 8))
 (segment (start 95.3925 92.3125) (end 95.08 92) (width 1) (layer "F.Cu") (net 5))
 (segment (start 136 81.9125) (end 136 83) (width 0.25) (layer "F.Cu") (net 2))
 (segment (start 138 82.5) (end 137.5 83) (width 0.25) (layer "F.Cu") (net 2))
 (segment (start 136 83) (end 136 84.175) (width 0.25) (layer "F.Cu") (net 2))
 (segment (start 137.5 83) (end 136 83) (width 0.25) (layer "F.Cu") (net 2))
 (segment (start 138 72.54) (end 138 82.5) (width 0.25) (layer "F.Cu") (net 2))
 (segment (start 133.65 88.85) (end 134 88.5) (width 0.25) (layer "F.Cu") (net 3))
 (segment (start 136 78) (end 134 76) (width 0.25) (layer "F.Cu") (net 3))
 (segment (start 130.665 72.665) (end 130.665 67.6) (width 0.25) (layer "F.Cu") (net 3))
 (segment (start 133 88.85) (end 133.65 88.85) (width 0.25) (layer "F.Cu") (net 3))
 (segment (start 136 80.0875) (end 136 78) (width 0.25) (layer "F.Cu") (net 3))
 (segment (start 134 88.5) (end 134 76) (width 0.25) (layer "F.Cu") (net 3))
 (segment (start 134 76) (end 130.665 72.665) (width 0.25) (layer "F.Cu") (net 3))
 (segment (start 136 86) (end 136 88) (width 0.25) (layer "F.Cu") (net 7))
 (segment (start 136 88) (end 133.85 90.15) (width 0.25) (layer "F.Cu") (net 7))
 (segment (start 133.85 90.15) (end 133 90.15) (width 0.25) (layer "F.Cu") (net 7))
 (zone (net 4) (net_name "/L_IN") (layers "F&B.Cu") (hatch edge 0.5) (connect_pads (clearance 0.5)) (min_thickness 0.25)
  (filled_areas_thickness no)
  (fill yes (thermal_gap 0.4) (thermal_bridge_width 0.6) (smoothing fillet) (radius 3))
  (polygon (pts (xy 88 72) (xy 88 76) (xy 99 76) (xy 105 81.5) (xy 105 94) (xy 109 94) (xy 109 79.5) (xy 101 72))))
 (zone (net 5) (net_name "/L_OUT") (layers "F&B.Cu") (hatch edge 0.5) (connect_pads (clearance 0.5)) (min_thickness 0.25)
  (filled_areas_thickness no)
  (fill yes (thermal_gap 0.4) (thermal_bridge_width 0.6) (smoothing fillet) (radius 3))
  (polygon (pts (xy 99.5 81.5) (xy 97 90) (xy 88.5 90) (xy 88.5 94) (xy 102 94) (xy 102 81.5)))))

